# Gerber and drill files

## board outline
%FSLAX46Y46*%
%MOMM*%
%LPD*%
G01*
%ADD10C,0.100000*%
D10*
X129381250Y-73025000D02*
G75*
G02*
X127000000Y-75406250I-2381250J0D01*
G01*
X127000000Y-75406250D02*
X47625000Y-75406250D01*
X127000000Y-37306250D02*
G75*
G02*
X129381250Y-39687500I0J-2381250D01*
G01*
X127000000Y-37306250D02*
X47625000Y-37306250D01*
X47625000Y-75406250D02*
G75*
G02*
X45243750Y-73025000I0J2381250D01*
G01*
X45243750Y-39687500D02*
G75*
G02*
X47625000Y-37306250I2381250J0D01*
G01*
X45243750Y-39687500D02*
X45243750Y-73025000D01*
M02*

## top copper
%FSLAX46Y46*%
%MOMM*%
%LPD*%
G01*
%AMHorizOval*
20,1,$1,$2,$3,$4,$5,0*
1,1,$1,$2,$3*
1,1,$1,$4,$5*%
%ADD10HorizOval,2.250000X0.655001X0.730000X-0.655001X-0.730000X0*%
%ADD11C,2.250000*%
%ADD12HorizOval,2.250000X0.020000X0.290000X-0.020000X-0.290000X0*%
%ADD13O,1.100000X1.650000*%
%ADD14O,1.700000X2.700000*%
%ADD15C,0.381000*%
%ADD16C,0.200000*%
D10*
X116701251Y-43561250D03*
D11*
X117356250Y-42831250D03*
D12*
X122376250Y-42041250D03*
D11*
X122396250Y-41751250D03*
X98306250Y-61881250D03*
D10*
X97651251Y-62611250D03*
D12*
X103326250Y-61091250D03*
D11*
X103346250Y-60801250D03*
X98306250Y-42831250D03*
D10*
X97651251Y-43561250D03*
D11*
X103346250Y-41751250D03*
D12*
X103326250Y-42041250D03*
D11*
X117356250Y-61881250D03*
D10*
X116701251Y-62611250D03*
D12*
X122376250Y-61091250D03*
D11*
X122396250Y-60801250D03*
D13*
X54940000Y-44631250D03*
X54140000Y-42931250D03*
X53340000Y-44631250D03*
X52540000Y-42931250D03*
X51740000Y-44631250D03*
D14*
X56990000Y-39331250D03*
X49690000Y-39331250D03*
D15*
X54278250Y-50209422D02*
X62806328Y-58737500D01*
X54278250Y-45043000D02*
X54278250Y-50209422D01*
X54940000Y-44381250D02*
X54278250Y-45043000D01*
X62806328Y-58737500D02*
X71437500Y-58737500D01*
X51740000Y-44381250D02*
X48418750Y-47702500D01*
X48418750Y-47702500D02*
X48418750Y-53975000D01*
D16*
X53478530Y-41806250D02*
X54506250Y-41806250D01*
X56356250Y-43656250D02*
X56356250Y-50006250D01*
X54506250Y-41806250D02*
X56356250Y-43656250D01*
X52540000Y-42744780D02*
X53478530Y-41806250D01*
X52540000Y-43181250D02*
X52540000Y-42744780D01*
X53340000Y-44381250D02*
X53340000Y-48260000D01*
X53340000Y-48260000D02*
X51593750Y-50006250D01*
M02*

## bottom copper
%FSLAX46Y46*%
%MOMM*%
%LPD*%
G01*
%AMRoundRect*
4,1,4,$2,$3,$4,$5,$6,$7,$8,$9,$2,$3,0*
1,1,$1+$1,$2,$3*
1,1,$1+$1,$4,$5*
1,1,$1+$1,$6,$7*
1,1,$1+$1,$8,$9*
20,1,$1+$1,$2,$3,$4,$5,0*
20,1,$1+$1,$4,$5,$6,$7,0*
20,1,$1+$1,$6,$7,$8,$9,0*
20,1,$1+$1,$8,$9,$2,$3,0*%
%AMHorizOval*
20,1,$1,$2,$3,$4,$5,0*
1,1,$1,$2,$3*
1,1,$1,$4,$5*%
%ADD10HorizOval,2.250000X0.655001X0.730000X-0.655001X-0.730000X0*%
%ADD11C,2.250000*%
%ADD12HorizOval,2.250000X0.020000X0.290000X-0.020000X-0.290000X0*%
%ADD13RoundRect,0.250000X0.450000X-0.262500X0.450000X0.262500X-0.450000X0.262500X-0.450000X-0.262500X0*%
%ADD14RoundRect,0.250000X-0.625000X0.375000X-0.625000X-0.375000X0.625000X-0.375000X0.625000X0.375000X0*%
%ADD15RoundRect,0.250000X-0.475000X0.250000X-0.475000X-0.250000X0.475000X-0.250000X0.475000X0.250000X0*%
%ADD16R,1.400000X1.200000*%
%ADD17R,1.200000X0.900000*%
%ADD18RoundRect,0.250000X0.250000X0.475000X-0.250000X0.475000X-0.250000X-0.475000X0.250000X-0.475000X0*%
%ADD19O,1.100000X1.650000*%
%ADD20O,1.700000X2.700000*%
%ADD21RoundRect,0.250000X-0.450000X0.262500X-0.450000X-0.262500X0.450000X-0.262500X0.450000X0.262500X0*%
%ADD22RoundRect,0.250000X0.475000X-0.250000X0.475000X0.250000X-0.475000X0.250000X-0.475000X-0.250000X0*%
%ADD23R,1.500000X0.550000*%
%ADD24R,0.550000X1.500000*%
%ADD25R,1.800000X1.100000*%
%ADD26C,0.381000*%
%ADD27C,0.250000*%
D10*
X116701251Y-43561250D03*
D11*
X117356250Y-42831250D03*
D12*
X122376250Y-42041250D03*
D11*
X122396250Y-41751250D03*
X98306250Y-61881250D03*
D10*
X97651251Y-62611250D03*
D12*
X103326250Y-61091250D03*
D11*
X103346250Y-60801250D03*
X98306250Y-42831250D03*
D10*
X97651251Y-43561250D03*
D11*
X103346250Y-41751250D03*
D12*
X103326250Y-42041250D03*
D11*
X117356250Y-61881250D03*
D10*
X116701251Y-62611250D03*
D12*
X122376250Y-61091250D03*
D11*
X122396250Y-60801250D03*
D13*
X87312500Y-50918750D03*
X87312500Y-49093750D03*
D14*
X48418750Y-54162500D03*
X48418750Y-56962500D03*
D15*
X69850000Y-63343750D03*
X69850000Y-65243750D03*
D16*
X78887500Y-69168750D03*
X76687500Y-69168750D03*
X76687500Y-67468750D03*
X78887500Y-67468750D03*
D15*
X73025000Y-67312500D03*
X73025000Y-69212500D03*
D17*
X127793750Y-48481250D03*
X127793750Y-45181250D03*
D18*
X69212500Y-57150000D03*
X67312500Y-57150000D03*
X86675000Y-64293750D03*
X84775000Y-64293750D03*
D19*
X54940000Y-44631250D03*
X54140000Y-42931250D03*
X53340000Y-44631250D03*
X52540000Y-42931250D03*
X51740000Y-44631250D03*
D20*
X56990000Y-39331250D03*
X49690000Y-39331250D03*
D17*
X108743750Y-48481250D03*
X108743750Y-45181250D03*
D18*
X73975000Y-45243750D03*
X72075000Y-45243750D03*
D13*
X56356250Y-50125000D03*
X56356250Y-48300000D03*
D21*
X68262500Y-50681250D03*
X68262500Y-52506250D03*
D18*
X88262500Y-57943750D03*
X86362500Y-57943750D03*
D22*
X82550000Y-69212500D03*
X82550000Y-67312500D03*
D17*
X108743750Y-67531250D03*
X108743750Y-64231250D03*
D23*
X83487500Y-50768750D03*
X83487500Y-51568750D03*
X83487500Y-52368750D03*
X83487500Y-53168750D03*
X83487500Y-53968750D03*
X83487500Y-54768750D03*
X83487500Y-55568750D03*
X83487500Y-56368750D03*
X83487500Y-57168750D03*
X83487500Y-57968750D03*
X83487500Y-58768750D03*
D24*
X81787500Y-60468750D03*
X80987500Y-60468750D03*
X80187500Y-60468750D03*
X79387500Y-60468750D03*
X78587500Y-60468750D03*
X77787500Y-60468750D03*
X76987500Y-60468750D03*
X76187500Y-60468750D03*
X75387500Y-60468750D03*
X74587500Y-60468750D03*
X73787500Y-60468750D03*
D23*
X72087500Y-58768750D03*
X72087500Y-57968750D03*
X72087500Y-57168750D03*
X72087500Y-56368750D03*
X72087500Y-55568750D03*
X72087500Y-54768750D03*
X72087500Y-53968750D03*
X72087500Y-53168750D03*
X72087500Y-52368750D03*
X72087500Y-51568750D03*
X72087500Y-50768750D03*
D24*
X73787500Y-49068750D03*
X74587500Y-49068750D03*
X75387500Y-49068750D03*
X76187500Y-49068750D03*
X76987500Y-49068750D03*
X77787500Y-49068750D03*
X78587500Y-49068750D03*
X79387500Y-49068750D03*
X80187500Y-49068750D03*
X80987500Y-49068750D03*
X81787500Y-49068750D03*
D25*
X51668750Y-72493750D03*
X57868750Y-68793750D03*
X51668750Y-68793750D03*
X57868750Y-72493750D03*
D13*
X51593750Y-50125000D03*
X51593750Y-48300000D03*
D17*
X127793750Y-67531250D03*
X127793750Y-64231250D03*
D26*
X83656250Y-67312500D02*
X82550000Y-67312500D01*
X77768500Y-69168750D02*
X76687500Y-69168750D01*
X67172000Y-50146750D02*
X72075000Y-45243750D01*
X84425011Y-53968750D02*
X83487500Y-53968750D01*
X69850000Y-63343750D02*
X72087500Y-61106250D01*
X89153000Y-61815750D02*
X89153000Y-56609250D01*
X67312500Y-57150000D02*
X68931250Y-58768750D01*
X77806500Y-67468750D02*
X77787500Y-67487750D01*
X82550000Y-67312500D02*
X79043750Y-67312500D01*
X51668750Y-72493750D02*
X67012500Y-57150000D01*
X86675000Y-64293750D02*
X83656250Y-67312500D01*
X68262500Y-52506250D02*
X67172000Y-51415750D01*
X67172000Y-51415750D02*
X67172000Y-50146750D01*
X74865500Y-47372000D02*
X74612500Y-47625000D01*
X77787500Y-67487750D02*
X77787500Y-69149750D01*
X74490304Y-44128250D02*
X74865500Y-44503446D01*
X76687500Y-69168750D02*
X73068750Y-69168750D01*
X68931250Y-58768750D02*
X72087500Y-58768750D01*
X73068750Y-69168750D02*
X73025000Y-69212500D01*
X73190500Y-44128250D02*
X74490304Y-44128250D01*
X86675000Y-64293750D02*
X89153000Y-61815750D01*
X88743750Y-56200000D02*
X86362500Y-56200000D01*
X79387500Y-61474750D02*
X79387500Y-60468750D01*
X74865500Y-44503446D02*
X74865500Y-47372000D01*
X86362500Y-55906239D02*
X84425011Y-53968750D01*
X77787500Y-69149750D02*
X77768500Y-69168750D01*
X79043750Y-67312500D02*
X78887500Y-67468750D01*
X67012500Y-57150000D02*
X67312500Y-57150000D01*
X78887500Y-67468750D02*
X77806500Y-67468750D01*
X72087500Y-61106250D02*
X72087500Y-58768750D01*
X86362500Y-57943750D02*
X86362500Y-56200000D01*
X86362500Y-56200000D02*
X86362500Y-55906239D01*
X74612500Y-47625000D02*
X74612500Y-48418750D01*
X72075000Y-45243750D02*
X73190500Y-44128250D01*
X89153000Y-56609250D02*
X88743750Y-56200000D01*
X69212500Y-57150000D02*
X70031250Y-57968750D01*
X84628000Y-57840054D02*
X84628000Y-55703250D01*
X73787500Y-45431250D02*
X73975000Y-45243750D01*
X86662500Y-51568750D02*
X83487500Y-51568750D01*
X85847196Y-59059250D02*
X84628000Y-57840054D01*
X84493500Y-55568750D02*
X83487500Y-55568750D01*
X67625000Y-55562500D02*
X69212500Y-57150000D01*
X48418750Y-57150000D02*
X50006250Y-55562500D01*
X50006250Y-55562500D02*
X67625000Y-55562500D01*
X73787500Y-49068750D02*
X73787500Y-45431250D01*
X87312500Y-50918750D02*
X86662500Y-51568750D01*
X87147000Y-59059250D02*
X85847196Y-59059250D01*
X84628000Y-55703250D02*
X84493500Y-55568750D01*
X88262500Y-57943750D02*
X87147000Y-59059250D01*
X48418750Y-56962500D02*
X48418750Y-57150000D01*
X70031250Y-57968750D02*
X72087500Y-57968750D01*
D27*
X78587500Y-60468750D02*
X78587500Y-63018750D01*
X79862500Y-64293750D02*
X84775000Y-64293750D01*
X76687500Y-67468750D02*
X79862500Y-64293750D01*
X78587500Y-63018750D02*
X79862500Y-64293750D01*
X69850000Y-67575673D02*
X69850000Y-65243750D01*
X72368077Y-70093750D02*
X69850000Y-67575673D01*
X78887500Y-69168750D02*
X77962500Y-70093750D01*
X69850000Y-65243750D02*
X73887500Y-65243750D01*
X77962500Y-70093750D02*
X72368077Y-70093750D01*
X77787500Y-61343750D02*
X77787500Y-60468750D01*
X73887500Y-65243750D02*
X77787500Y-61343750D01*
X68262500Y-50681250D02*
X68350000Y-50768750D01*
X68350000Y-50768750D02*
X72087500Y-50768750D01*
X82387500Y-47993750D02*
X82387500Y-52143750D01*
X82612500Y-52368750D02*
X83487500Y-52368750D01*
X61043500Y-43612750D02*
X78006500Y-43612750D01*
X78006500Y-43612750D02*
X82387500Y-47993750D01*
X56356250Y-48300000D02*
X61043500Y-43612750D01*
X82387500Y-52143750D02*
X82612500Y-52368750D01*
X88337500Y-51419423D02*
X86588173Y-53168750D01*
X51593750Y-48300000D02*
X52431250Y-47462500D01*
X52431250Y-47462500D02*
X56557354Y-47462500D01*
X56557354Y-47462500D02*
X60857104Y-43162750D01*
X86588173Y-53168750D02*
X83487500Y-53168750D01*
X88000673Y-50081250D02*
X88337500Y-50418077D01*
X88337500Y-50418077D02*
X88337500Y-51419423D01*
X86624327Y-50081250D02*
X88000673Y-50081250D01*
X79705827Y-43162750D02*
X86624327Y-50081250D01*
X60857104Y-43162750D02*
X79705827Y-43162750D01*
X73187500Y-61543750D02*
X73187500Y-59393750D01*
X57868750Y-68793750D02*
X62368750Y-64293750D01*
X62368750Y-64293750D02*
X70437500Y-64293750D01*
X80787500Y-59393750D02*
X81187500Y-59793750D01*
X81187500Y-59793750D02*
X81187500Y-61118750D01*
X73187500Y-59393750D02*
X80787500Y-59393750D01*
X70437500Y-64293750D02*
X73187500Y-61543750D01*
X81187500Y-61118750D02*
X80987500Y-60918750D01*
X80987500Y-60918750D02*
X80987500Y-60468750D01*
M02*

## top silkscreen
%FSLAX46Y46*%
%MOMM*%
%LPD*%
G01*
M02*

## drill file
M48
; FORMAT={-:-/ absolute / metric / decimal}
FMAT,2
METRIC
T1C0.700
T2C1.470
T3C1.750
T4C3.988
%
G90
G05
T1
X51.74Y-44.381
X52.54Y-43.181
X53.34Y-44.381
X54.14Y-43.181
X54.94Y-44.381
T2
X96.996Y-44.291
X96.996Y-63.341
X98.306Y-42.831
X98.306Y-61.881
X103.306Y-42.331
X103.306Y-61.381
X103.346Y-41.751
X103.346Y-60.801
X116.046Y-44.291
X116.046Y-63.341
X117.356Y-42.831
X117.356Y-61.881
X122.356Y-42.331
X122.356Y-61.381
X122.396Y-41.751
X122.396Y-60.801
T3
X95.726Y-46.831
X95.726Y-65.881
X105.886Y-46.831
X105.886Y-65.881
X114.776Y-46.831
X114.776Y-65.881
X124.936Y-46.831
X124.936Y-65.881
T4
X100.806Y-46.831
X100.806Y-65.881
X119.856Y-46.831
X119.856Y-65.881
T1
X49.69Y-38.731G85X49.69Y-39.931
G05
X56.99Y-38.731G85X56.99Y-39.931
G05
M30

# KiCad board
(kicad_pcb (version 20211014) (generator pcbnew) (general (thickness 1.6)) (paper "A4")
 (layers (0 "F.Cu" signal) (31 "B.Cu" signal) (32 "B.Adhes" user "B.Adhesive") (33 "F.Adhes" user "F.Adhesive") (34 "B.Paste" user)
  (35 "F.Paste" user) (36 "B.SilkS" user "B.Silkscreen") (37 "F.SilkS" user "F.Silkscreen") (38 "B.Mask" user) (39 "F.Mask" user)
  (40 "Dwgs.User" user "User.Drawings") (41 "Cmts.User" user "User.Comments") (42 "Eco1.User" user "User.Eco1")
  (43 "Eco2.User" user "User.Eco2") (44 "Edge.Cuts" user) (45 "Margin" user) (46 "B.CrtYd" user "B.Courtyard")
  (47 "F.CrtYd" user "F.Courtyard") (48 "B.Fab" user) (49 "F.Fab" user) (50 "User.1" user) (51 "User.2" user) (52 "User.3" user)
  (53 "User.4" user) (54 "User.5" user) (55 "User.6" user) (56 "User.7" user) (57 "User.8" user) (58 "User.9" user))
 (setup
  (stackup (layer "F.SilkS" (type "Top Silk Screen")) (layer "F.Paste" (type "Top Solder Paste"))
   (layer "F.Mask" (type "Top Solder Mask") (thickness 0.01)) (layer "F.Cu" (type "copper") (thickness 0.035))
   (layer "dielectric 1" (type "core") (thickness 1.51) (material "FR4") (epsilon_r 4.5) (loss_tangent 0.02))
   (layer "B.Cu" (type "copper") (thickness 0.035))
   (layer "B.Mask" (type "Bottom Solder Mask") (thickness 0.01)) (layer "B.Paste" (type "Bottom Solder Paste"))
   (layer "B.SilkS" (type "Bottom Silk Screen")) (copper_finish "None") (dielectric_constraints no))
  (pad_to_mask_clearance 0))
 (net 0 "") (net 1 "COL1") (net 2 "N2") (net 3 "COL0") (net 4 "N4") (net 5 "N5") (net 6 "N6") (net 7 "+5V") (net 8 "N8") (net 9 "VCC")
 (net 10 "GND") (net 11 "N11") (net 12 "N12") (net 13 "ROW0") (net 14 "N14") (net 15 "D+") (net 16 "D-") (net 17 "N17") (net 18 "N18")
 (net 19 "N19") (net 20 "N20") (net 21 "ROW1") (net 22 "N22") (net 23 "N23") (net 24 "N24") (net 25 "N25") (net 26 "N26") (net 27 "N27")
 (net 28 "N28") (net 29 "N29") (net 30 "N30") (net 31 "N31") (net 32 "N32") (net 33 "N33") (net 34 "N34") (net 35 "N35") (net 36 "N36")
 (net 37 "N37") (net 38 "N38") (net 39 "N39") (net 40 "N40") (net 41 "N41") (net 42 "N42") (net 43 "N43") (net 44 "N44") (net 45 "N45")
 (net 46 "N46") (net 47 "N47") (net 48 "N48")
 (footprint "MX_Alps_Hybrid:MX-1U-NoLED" (layer "F.Cu") (at 119.85625 46.83125)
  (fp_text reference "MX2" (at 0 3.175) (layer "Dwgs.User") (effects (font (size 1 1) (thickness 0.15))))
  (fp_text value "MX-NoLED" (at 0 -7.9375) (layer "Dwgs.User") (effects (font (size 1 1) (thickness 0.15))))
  (pad "" np_thru_hole circle locked (at 5.08 0 48.0996) (size 1.75 1.75) (drill 1.75) (layers *.Cu *.Mask))
  (pad "" np_thru_hole circle locked (at 0 0) (size 3.9878 3.9878) (drill 3.9878) (layers *.Cu *.Mask))
  (pad "" np_thru_hole circle locked (at -5.08 0 48.0996) (size 1.75 1.75) (drill 1.75) (layers *.Cu *.Mask))
  (pad "1" thru_hole oval locked (at -3.81 -2.54 48.0996) (size 4.211556 2.25) (drill 1.47 (offset 0.980778 0)) (layers *.Cu "B.Mask")
   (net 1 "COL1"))
  (pad "1" thru_hole circle locked (at -2.5 -4) (size 2.25 2.25) (drill 1.47) (layers *.Cu "B.Mask") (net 1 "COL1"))
  (pad "2" thru_hole oval locked (at 2.5 -4.5 86.0548) (size 2.831378 2.25) (drill 1.47 (offset 0.290689 0)) (layers *.Cu "B.Mask")
   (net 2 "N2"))
  (pad "2" thru_hole circle locked (at 2.54 -5.08) (size 2.25 2.25) (drill 1.47) (layers *.Cu "B.Mask") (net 2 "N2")))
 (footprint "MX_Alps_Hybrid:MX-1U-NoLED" (layer "F.Cu") (at 100.80625 65.88125)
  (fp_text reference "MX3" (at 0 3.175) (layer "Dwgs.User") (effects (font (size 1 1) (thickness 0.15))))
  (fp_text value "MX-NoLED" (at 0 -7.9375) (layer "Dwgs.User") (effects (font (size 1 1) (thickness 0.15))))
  (pad "" np_thru_hole circle locked (at 5.08 0 48.0996) (size 1.75 1.75) (drill 1.75) (layers *.Cu *.Mask))
  (pad "" np_thru_hole circle locked (at 0 0) (size 3.9878 3.9878) (drill 3.9878) (layers *.Cu *.Mask))
  (pad "" np_thru_hole circle locked (at -5.08 0 48.0996) (size 1.75 1.75) (drill 1.75) (layers *.Cu *.Mask))
  (pad "1" thru_hole circle locked (at -2.5 -4) (size 2.25 2.25) (drill 1.47) (layers *.Cu "B.Mask") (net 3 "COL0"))
  (pad "1" thru_hole oval locked (at -3.81 -2.54 48.0996) (size 4.211556 2.25) (drill 1.47 (offset 0.980778 0)) (layers *.Cu "B.Mask")
   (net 3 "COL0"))
  (pad "2" thru_hole oval locked (at 2.5 -4.5 86.0548) (size 2.831378 2.25) (drill 1.47 (offset 0.290689 0)) (layers *.Cu "B.Mask")
   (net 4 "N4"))
  (pad "2" thru_hole circle locked (at 2.54 -5.08) (size 2.25 2.25) (drill 1.47) (layers *.Cu "B.Mask") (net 4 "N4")))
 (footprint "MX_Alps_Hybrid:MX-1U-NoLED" (layer "F.Cu") (at 100.80625 46.83125)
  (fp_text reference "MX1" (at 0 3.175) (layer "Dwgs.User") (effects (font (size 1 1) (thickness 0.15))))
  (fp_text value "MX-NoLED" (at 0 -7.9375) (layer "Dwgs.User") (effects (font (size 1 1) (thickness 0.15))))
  (pad "" np_thru_hole circle locked (at 0 0) (size 3.9878 3.9878) (drill 3.9878) (layers *.Cu *.Mask))
  (pad "" np_thru_hole circle locked (at -5.08 0 48.0996) (size 1.75 1.75) (drill 1.75) (layers *.Cu *.Mask))
  (pad "" np_thru_hole circle locked (at 5.08 0 48.0996) (size 1.75 1.75) (drill 1.75) (layers *.Cu *.Mask))
  (pad "1" thru_hole circle locked (at -2.5 -4) (size 2.25 2.25) (drill 1.47) (layers *.Cu "B.Mask") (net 3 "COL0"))
  (pad "1" thru_hole oval locked (at -3.81 -2.54 48.0996) (size 4.211556 2.25) (drill 1.47 (offset 0.980778 0)) (layers *.Cu "B.Mask")
   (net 3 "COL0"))
  (pad "2" thru_hole circle locked (at 2.54 -5.08) (size 2.25 2.25) (drill 1.47) (layers *.Cu "B.Mask") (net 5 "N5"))
  (pad "2" thru_hole oval locked (at 2.5 -4.5 86.0548) (size 2.831378 2.25) (drill 1.47 (offset 0.290689 0)) (layers *.Cu "B.Mask")
   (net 5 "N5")))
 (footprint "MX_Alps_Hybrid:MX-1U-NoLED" (layer "F.Cu") (at 119.85625 65.88125)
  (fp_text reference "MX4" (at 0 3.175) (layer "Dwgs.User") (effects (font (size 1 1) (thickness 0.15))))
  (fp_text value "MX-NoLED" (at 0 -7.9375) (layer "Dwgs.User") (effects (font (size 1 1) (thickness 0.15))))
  (pad "" np_thru_hole circle locked (at 5.08 0 48.0996) (size 1.75 1.75) (drill 1.75) (layers *.Cu *.Mask))
  (pad "" np_thru_hole circle locked (at -5.08 0 48.0996) (size 1.75 1.75) (drill 1.75) (layers *.Cu *.Mask))
  (pad "" np_thru_hole circle locked (at 0 0) (size 3.9878 3.9878) (drill 3.9878) (layers *.Cu *.Mask))
  (pad "1" thru_hole circle locked (at -2.5 -4) (size 2.25 2.25) (drill 1.47) (layers *.Cu "B.Mask") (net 1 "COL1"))
  (pad "1" thru_hole oval locked (at -3.81 -2.54 48.0996) (size 4.211556 2.25) (drill 1.47 (offset 0.980778 0)) (layers *.Cu "B.Mask")
   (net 1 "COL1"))
  (pad "2" thru_hole oval locked (at 2.5 -4.5 86.0548) (size 2.831378 2.25) (drill 1.47 (offset 0.290689 0)) (layers *.Cu "B.Mask")
   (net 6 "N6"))
  (pad "2" thru_hole circle locked (at 2.54 -5.08) (size 2.25 2.25) (drill 1.47) (layers *.Cu "B.Mask") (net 6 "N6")))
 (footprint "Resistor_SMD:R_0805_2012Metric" (layer "B.Cu") (at 87.3125 50.00625 90)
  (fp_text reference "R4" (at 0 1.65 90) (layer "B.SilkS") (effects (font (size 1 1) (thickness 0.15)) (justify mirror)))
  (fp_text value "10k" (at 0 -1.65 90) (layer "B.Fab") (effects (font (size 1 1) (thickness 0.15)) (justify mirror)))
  (pad "1" smd roundrect (at -0.9125 0 90) (size 1.025 1.4) (layers "B.Cu" "B.Paste" "B.Mask") (roundrect_rratio 0.243902) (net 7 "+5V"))
  (pad "2" smd roundrect (at 0.9125 0 90) (size 1.025 1.4) (layers "B.Cu" "B.Paste" "B.Mask") (roundrect_rratio 0.243902) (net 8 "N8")))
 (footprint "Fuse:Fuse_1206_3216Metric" (layer "B.Cu") (at 48.41875 55.5625 -90)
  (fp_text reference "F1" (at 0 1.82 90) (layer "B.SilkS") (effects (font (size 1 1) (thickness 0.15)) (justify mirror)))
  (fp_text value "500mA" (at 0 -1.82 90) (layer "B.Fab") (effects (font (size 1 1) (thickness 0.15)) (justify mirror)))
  (pad "1" smd roundrect (at -1.4 0 270) (size 1.25 1.75) (layers "B.Cu" "B.Paste" "B.Mask") (roundrect_rratio 0.2) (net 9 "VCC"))
  (pad "2" smd roundrect (at 1.4 0 270) (size 1.25 1.75) (layers "B.Cu" "B.Paste" "B.Mask") (roundrect_rratio 0.2) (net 7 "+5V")))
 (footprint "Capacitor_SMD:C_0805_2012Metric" (layer "B.Cu") (at 69.85 64.29375 -90)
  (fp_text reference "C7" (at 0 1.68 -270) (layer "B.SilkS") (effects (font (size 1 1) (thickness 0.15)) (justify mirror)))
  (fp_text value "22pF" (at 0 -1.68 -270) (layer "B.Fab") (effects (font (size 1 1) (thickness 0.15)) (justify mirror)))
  (pad "1" smd roundrect (at -0.95 0 270) (size 1 1.45) (layers "B.Cu" "B.Paste" "B.Mask") (roundrect_rratio 0.25) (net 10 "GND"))
  (pad "2" smd roundrect (at 0.95 0 270) (size 1 1.45) (layers "B.Cu" "B.Paste" "B.Mask") (roundrect_rratio 0.25) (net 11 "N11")))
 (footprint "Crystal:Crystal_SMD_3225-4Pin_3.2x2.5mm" (layer "B.Cu") (at 77.7875 68.31875 180)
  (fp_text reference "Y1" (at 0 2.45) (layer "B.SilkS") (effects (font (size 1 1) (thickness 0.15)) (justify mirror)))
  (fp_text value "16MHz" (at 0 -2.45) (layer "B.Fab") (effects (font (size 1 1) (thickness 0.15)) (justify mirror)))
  (pad "1" smd rect (at -1.1 -0.85 180) (size 1.4 1.2) (layers "B.Cu" "B.Paste" "B.Mask") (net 11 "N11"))
  (pad "2" smd rect (at 1.1 -0.85 180) (size 1.4 1.2) (layers "B.Cu" "B.Paste" "B.Mask") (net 10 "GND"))
  (pad "3" smd rect (at 1.1 0.85 180) (size 1.4 1.2) (layers "B.Cu" "B.Paste" "B.Mask") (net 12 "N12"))
  (pad "4" smd rect (at -1.1 0.85 180) (size 1.4 1.2) (layers "B.Cu" "B.Paste" "B.Mask") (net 10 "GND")))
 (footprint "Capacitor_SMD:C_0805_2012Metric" (layer "B.Cu") (at 73.025 68.2625 -90)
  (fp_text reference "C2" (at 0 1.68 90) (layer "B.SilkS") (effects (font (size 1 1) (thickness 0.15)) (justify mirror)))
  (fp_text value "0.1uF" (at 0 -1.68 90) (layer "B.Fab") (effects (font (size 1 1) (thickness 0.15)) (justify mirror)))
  (pad "1" smd roundrect (at -0.95 0 270) (size 1 1.45) (layers "B.Cu" "B.Paste" "B.Mask") (roundrect_rratio 0.25) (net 7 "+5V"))
  (pad "2" smd roundrect (at 0.95 0 270) (size 1 1.45) (layers "B.Cu" "B.Paste" "B.Mask") (roundrect_rratio 0.25) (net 10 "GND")))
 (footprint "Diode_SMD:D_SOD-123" (layer "B.Cu") (at 127.79375 46.83125 90)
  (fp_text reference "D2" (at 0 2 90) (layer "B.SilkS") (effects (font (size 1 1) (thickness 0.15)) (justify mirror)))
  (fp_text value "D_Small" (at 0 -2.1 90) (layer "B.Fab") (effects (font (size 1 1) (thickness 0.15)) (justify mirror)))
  (pad "1" smd rect (at -1.65 0 90) (size 0.9 1.2) (layers "B.Cu" "B.Paste" "B.Mask") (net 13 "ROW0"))
  (pad "2" smd rect (at 1.65 0 90) (size 0.9 1.2) (layers "B.Cu" "B.Paste" "B.Mask") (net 2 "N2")))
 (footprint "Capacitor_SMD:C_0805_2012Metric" (layer "B.Cu") (at 68.2625 57.15 180)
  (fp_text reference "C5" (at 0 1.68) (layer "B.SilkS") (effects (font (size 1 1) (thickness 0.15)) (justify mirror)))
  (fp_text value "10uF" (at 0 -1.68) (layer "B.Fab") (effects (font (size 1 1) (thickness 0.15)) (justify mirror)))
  (pad "1" smd roundrect (at -0.95 0 180) (size 1 1.45) (layers "B.Cu" "B.Paste" "B.Mask") (roundrect_rratio 0.25) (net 7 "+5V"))
  (pad "2" smd roundrect (at 0.95 0 180) (size 1 1.45) (layers "B.Cu" "B.Paste" "B.Mask") (roundrect_rratio 0.25) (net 10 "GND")))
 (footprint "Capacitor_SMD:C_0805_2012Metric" (layer "B.Cu") (at 85.725 64.29375 180)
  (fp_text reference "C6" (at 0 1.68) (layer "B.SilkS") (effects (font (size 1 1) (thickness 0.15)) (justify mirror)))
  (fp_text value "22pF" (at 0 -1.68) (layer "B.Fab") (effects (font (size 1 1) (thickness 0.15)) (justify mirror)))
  (pad "1" smd roundrect (at -0.95 0 180) (size 1 1.45) (layers "B.Cu" "B.Paste" "B.Mask") (roundrect_rratio 0.25) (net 10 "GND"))
  (pad "2" smd roundrect (at 0.95 0 180) (size 1 1.45) (layers "B.Cu" "B.Paste" "B.Mask") (roundrect_rratio 0.25) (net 12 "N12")))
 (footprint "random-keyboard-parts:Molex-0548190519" (layer "B.Cu") (at 53.34 37.58125 -90)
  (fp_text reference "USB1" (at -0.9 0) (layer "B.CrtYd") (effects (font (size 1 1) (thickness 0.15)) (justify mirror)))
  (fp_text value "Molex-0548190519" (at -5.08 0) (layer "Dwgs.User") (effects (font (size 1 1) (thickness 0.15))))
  (pad "1" thru_hole oval locked (at 6.8 -1.6 270) (size 1.65 1.1) (drill oval 0.7 (offset 0.25 0)) (layers *.Cu "F.Mask") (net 10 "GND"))
  (pad "2" thru_hole oval locked (at 5.6 -0.8 90) (size 1.65 1.1) (drill oval 0.7 (offset 0.25 0)) (layers *.Cu "F.Mask") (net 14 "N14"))
  (pad "3" thru_hole oval locked (at 6.8 0 270) (size 1.65 1.1) (drill oval 0.7 (offset 0.25 0)) (layers *.Cu "F.Mask") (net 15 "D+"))
  (pad "4" thru_hole oval locked (at 5.6 0.8 90) (size 1.65 1.1) (drill oval 0.7 (offset 0.25 0)) (layers *.Cu "F.Mask") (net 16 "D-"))
  (pad "5" thru_hole oval locked (at 6.8 1.6 270) (size 1.65 1.1) (drill oval 0.7 (offset 0.25 0)) (layers *.Cu "F.Mask") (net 9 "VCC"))
  (pad "6" thru_hole oval locked (at 1.75 -3.65 270) (size 2.7 1.7) (drill oval 1.9 0.7) (layers *.Cu *.Mask) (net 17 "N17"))
  (pad "6" thru_hole oval locked (at 1.75 3.65 270) (size 2.7 1.7) (drill oval 1.9 0.7) (layers *.Cu *.Mask) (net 17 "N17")))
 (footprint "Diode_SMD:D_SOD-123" (layer "B.Cu") (at 108.74375 46.83125 90)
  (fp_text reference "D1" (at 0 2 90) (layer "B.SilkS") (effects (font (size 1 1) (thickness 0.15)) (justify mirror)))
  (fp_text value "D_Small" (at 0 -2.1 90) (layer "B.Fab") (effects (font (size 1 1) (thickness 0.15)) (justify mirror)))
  (pad "1" smd rect (at -1.65 0 90) (size 0.9 1.2) (layers "B.Cu" "B.Paste" "B.Mask") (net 13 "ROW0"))
  (pad "2" smd rect (at 1.65 0 90) (size 0.9 1.2) (layers "B.Cu" "B.Paste" "B.Mask") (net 5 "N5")))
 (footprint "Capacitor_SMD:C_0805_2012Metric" (layer "B.Cu") (at 73.025 45.24375 180)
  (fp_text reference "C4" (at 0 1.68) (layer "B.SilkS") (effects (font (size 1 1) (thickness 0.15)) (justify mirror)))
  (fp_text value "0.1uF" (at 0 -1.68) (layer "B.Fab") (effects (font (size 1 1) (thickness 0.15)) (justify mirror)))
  (pad "1" smd roundrect (at -0.95 0 180) (size 1 1.45) (layers "B.Cu" "B.Paste" "B.Mask") (roundrect_rratio 0.25) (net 7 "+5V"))
  (pad "2" smd roundrect (at 0.95 0 180) (size 1 1.45) (layers "B.Cu" "B.Paste" "B.Mask") (roundrect_rratio 0.25) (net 10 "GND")))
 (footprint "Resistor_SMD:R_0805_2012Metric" (layer "B.Cu") (at 56.35625 49.2125 90)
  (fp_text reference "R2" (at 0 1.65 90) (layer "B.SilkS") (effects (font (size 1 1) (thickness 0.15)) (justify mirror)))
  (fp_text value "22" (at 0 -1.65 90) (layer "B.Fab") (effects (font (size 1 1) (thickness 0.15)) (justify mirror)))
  (pad "1" smd roundrect (at -0.9125 0 90) (size 1.025 1.4) (layers "B.Cu" "B.Paste" "B.Mask") (roundrect_rratio 0.243902) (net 16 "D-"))
  (pad "2" smd roundrect (at 0.9125 0 90) (size 1.025 1.4) (layers "B.Cu" "B.Paste" "B.Mask") (roundrect_rratio 0.243902) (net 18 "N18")))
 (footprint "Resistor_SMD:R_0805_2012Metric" (layer "B.Cu") (at 68.2625 51.59375 -90)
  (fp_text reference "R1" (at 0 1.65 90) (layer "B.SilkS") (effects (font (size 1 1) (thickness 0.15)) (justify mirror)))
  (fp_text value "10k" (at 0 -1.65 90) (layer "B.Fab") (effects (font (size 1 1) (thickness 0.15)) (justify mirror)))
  (pad "1" smd roundrect (at -0.9125 0 270) (size 1.025 1.4) (layers "B.Cu" "B.Paste" "B.Mask") (roundrect_rratio 0.243902) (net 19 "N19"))
  (pad "2" smd roundrect (at 0.9125 0 270) (size 1.025 1.4) (layers "B.Cu" "B.Paste" "B.Mask") (roundrect_rratio 0.243902) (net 10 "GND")))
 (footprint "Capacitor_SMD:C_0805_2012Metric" (layer "B.Cu") (at 87.3125 57.94375 180)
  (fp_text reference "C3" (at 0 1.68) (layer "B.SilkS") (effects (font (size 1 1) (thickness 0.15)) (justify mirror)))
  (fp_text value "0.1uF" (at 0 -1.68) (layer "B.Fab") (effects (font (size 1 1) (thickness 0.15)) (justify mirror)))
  (pad "1" smd roundrect (at -0.95 0 180) (size 1 1.45) (layers "B.Cu" "B.Paste" "B.Mask") (roundrect_rratio 0.25) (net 7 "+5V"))
  (pad "2" smd roundrect (at 0.95 0 180) (size 1 1.45) (layers "B.Cu" "B.Paste" "B.Mask") (roundrect_rratio 0.25) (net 10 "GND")))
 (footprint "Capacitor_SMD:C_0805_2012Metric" (layer "B.Cu") (at 82.55 68.2625 90)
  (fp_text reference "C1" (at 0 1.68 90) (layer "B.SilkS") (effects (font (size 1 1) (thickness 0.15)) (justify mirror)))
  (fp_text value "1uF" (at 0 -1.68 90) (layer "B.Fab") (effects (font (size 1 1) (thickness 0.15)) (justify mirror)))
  (pad "1" smd roundrect (at -0.95 0 90) (size 1 1.45) (layers "B.Cu" "B.Paste" "B.Mask") (roundrect_rratio 0.25) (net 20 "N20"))
  (pad "2" smd roundrect (at 0.95 0 90) (size 1 1.45) (layers "B.Cu" "B.Paste" "B.Mask") (roundrect_rratio 0.25) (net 10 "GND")))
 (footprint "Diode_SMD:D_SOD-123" (layer "B.Cu") (at 108.74375 65.88125 90)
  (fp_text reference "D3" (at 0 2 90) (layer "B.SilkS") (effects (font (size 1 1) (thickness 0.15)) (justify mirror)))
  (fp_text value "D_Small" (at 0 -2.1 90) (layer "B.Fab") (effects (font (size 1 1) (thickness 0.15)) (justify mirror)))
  (pad "1" smd rect (at -1.65 0 90) (size 0.9 1.2) (layers "B.Cu" "B.Paste" "B.Mask") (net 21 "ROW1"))
  (pad "2" smd rect (at 1.65 0 90) (size 0.9 1.2) (layers "B.Cu" "B.Paste" "B.Mask") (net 4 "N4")))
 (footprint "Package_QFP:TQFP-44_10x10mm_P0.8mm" (layer "B.Cu") (at 77.7875 54.76875 180)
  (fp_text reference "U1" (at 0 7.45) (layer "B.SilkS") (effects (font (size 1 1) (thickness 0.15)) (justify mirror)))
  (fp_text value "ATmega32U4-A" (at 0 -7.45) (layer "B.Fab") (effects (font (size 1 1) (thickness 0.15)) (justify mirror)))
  (pad "1" smd rect (at -5.7 4 180) (size 1.5 0.55) (layers "B.Cu" "B.Paste" "B.Mask") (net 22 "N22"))
  (pad "2" smd rect (at -5.7 3.2 180) (size 1.5 0.55) (layers "B.Cu" "B.Paste" "B.Mask") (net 7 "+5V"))
  (pad "3" smd rect (at -5.7 2.4 180) (size 1.5 0.55) (layers "B.Cu" "B.Paste" "B.Mask") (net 18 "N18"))
  (pad "4" smd rect (at -5.7 1.6 180) (size 1.5 0.55) (layers "B.Cu" "B.Paste" "B.Mask") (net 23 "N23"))
  (pad "5" smd rect (at -5.7 0.8 180) (size 1.5 0.55) (layers "B.Cu" "B.Paste" "B.Mask") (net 10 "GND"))
  (pad "6" smd rect (at -5.7 0 180) (size 1.5 0.55) (layers "B.Cu" "B.Paste" "B.Mask") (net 20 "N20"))
  (pad "7" smd rect (at -5.7 -0.8 180) (size 1.5 0.55) (layers "B.Cu" "B.Paste" "B.Mask") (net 7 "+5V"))
  (pad "8" smd rect (at -5.7 -1.6 180) (size 1.5 0.55) (layers "B.Cu" "B.Paste" "B.Mask") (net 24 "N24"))
  (pad "9" smd rect (at -5.7 -2.4 180) (size 1.5 0.55) (layers "B.Cu" "B.Paste" "B.Mask") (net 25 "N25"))
  (pad "10" smd rect (at -5.7 -3.2 180) (size 1.5 0.55) (layers "B.Cu" "B.Paste" "B.Mask") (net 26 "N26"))
  (pad "11" smd rect (at -5.7 -4 180) (size 1.5 0.55) (layers "B.Cu" "B.Paste" "B.Mask") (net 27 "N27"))
  (pad "12" smd rect (at -4 -5.7 90) (size 1.5 0.55) (layers "B.Cu" "B.Paste" "B.Mask") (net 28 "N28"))
  (pad "13" smd rect (at -3.2 -5.7 90) (size 1.5 0.55) (layers "B.Cu" "B.Paste" "B.Mask") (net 8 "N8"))
  (pad "14" smd rect (at -2.4 -5.7 90) (size 1.5 0.55) (layers "B.Cu" "B.Paste" "B.Mask") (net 7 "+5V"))
  (pad "15" smd rect (at -1.6 -5.7 90) (size 1.5 0.55) (layers "B.Cu" "B.Paste" "B.Mask") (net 10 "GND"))
  (pad "16" smd rect (at -0.8 -5.7 90) (size 1.5 0.55) (layers "B.Cu" "B.Paste" "B.Mask") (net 12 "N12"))
  (pad "17" smd rect (at 0 -5.7 90) (size 1.5 0.55) (layers "B.Cu" "B.Paste" "B.Mask") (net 11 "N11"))
  (pad "18" smd rect (at 0.8 -5.7 90) (size 1.5 0.55) (layers "B.Cu" "B.Paste" "B.Mask") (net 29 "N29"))
  (pad "19" smd rect (at 1.6 -5.7 90) (size 1.5 0.55) (layers "B.Cu" "B.Paste" "B.Mask") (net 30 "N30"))
  (pad "20" smd rect (at 2.4 -5.7 90) (size 1.5 0.55) (layers "B.Cu" "B.Paste" "B.Mask") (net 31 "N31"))
  (pad "21" smd rect (at 3.2 -5.7 90) (size 1.5 0.55) (layers "B.Cu" "B.Paste" "B.Mask") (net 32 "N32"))
  (pad "22" smd rect (at 4 -5.7 90) (size 1.5 0.55) (layers "B.Cu" "B.Paste" "B.Mask") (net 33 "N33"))
  (pad "23" smd rect (at 5.7 -4 180) (size 1.5 0.55) (layers "B.Cu" "B.Paste" "B.Mask") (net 10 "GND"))
  (pad "24" smd rect (at 5.7 -3.2 180) (size 1.5 0.55) (layers "B.Cu" "B.Paste" "B.Mask") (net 7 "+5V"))
  (pad "25" smd rect (at 5.7 -2.4 180) (size 1.5 0.55) (layers "B.Cu" "B.Paste" "B.Mask") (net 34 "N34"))
  (pad "26" smd rect (at 5.7 -1.6 180) (size 1.5 0.55) (layers "B.Cu" "B.Paste" "B.Mask") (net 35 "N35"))
  (pad "27" smd rect (at 5.7 -0.8 180) (size 1.5 0.55) (layers "B.Cu" "B.Paste" "B.Mask") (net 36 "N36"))
  (pad "28" smd rect (at 5.7 0 180) (size 1.5 0.55) (layers "B.Cu" "B.Paste" "B.Mask") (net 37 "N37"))
  (pad "29" smd rect (at 5.7 0.8 180) (size 1.5 0.55) (layers "B.Cu" "B.Paste" "B.Mask") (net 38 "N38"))
  (pad "30" smd rect (at 5.7 1.6 180) (size 1.5 0.55) (layers "B.Cu" "B.Paste" "B.Mask") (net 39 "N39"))
  (pad "31" smd rect (at 5.7 2.4 180) (size 1.5 0.55) (layers "B.Cu" "B.Paste" "B.Mask") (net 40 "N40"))
  (pad "32" smd rect (at 5.7 3.2 180) (size 1.5 0.55) (layers "B.Cu" "B.Paste" "B.Mask") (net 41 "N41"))
  (pad "33" smd rect (at 5.7 4 180) (size 1.5 0.55) (layers "B.Cu" "B.Paste" "B.Mask") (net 19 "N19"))
  (pad "34" smd rect (at 4 5.7 90) (size 1.5 0.55) (layers "B.Cu" "B.Paste" "B.Mask") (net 7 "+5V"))
  (pad "35" smd rect (at 3.2 5.7 90) (size 1.5 0.55) (layers "B.Cu" "B.Paste" "B.Mask") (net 10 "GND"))
  (pad "36" smd rect (at 2.4 5.7 90) (size 1.5 0.55) (layers "B.Cu" "B.Paste" "B.Mask") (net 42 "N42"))
  (pad "37" smd rect (at 1.6 5.7 90) (size 1.5 0.55) (layers "B.Cu" "B.Paste" "B.Mask") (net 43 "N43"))
  (pad "38" smd rect (at 0.8 5.7 90) (size 1.5 0.55) (layers "B.Cu" "B.Paste" "B.Mask") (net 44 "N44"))
  (pad "39" smd rect (at 0 5.7 90) (size 1.5 0.55) (layers "B.Cu" "B.Paste" "B.Mask") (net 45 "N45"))
  (pad "40" smd rect (at -0.8 5.7 90) (size 1.5 0.55) (layers "B.Cu" "B.Paste" "B.Mask") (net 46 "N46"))
  (pad "41" smd rect (at -1.6 5.7 90) (size 1.5 0.55) (layers "B.Cu" "B.Paste" "B.Mask") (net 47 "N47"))
  (pad "42" smd rect (at -2.4 5.7 90) (size 1.5 0.55) (layers "B.Cu" "B.Paste" "B.Mask") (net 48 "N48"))
  (pad "43" smd rect (at -3.2 5.7 90) (size 1.5 0.55) (layers "B.Cu" "B.Paste" "B.Mask") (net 10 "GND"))
  (pad "44" smd rect (at -4 5.7 90) (size 1.5 0.55) (layers "B.Cu" "B.Paste" "B.Mask") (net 7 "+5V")))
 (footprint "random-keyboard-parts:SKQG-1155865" (layer "B.Cu") (at 54.76875 70.64375 180)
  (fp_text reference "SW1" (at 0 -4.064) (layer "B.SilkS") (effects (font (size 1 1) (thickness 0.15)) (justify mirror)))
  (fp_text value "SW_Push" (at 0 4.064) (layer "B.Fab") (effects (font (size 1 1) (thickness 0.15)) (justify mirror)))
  (pad "1" smd rect locked (at 3.1 -1.85 180) (size 1.8 1.1) (layers "B.Cu" "B.Paste" "B.Mask") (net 10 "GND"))
  (pad "2" smd rect locked (at -3.1 1.85 180) (size 1.8 1.1) (layers "B.Cu" "B.Paste" "B.Mask") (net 8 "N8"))
  (pad "3" smd rect locked (at 3.1 1.85 180) (size 1.8 1.1) (layers "B.Cu" "B.Paste" "B.Mask"))
  (pad "4" smd rect locked (at -3.1 -1.85 180) (size 1.8 1.1) (layers "B.Cu" "B.Paste" "B.Mask")))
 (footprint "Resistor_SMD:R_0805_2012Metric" (layer "B.Cu") (at 51.59375 49.2125 90)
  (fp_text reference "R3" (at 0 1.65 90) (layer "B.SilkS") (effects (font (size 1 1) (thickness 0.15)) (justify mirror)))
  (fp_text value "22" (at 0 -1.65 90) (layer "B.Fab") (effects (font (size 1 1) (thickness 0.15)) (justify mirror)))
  (pad "1" smd roundrect (at -0.9125 0 90) (size 1.025 1.4) (layers "B.Cu" "B.Paste" "B.Mask") (roundrect_rratio 0.243902) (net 15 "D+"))
  (pad "2" smd roundrect (at 0.9125 0 90) (size 1.025 1.4) (layers "B.Cu" "B.Paste" "B.Mask") (roundrect_rratio 0.243902) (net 23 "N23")))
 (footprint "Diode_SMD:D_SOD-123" (layer "B.Cu") (at 127.79375 65.88125 90)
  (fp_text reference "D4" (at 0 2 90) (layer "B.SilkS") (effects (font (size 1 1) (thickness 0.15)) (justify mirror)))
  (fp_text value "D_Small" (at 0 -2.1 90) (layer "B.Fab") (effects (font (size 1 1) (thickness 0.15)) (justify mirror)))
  (pad "1" smd rect (at -1.65 0 90) (size 0.9 1.2) (layers "B.Cu" "B.Paste" "B.Mask") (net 21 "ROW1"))
  (pad "2" smd rect (at 1.65 0 90) (size 0.9 1.2) (layers "B.Cu" "B.Paste" "B.Mask") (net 6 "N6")))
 (gr_arc (start 129.38125 73.025) (mid 128.683798 74.708798) (end 127 75.40625) (layer "Edge.Cuts") (width 0.1))
 (gr_line (start 127 75.40625) (end 47.625 75.40625) (layer "Edge.Cuts") (width 0.1))
 (gr_arc (start 127 37.30625) (mid 128.683798 38.003702) (end 129.38125 39.6875) (layer "Edge.Cuts") (width 0.1))
 (gr_line (start 127 37.30625) (end 47.625 37.30625) (layer "Edge.Cuts") (width 0.1))
 (gr_arc (start 47.625 75.40625) (mid 45.941202 74.708798) (end 45.24375 73.025) (layer "Edge.Cuts") (width 0.1))
 (gr_arc (start 45.24375 39.6875) (mid 45.941202 38.003702) (end 47.625 37.30625) (layer "Edge.Cuts") (width 0.1))
 (gr_line (start 45.24375 39.6875) (end 45.24375 73.025) (layer "Edge.Cuts") (width 0.1))
 (segment (start 54.27825 50.209422) (end 62.806328 58.7375) (width 0.381) (layer "F.Cu") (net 10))
 (segment (start 54.27825 45.043) (end 54.27825 50.209422) (width 0.381) (layer "F.Cu") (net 10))
 (segment (start 54.94 44.38125) (end 54.27825 45.043) (width 0.381) (layer "F.Cu") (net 10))
 (segment (start 62.806328 58.7375) (end 71.4375 58.7375) (width 0.381) (layer "F.Cu") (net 10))
 (segment (start 83.65625 67.3125) (end 82.55 67.3125) (width 0.381) (layer "B.Cu") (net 10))
 (segment (start 77.7685 69.16875) (end 76.6875 69.16875) (width 0.381) (layer "B.Cu") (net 10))
 (segment (start 67.172 50.14675) (end 72.075 45.24375) (width 0.381) (layer "B.Cu") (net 10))
 (segment (start 84.425011 53.96875) (end 83.4875 53.96875) (width 0.381) (layer "B.Cu") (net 10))
 (segment (start 69.85 63.34375) (end 72.0875 61.10625) (width 0.381) (layer "B.Cu") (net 10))
 (segment (start 89.153 61.81575) (end 89.153 56.60925) (width 0.381) (layer "B.Cu") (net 10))
 (segment (start 67.3125 57.15) (end 68.93125 58.76875) (width 0.381) (layer "B.Cu") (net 10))
 (segment (start 77.8065 67.46875) (end 77.7875 67.48775) (width 0.381) (layer "B.Cu") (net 10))
 (segment (start 82.55 67.3125) (end 79.04375 67.3125) (width 0.381) (layer "B.Cu") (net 10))
 (segment (start 51.66875 72.49375) (end 67.0125 57.15) (width 0.381) (layer "B.Cu") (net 10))
 (segment (start 86.675 64.29375) (end 83.65625 67.3125) (width 0.381) (layer "B.Cu") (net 10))
 (segment (start 68.2625 52.50625) (end 67.172 51.41575) (width 0.381) (layer "B.Cu") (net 10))
 (segment (start 67.172 51.41575) (end 67.172 50.14675) (width 0.381) (layer "B.Cu") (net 10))
 (segment (start 74.8655 47.372) (end 74.6125 47.625) (width 0.381) (layer "B.Cu") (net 10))
 (segment (start 77.7875 67.48775) (end 77.7875 69.14975) (width 0.381) (layer "B.Cu") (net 10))
 (segment (start 74.490304 44.12825) (end 74.8655 44.503446) (width 0.381) (layer "B.Cu") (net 10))
 (segment (start 76.6875 69.16875) (end 73.06875 69.16875) (width 0.381) (layer "B.Cu") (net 10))
 (segment (start 68.93125 58.76875) (end 72.0875 58.76875) (width 0.381) (layer "B.Cu") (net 10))
 (segment (start 73.06875 69.16875) (end 73.025 69.2125) (width 0.381) (layer "B.Cu") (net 10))
 (segment (start 73.1905 44.12825) (end 74.490304 44.12825) (width 0.381) (layer "B.Cu") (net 10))
 (segment (start 86.675 64.29375) (end 89.153 61.81575) (width 0.381) (layer "B.Cu") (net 10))
 (segment (start 88.74375 56.2) (end 86.3625 56.2) (width 0.381) (layer "B.Cu") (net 10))
 (segment (start 79.3875 61.47475) (end 79.3875 60.46875) (width 0.381) (layer "B.Cu") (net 10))
 (segment (start 74.8655 44.503446) (end 74.8655 47.372) (width 0.381) (layer "B.Cu") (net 10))
 (segment (start 86.3625 55.906239) (end 84.425011 53.96875) (width 0.381) (layer "B.Cu") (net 10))
 (segment (start 77.7875 69.14975) (end 77.7685 69.16875) (width 0.381) (layer "B.Cu") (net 10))
 (segment (start 79.04375 67.3125) (end 78.8875 67.46875) (width 0.381) (layer "B.Cu") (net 10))
 (segment (start 67.0125 57.15) (end 67.3125 57.15) (width 0.381) (layer "B.Cu") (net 10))
 (segment (start 78.8875 67.46875) (end 77.8065 67.46875) (width 0.381) (layer "B.Cu") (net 10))
 (segment (start 72.0875 61.10625) (end 72.0875 58.76875) (width 0.381) (layer "B.Cu") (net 10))
 (segment (start 86.3625 57.94375) (end 86.3625 56.2) (width 0.381) (layer "B.Cu") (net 10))
 (segment (start 86.3625 56.2) (end 86.3625 55.906239) (width 0.381) (layer "B.Cu") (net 10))
 (segment (start 74.6125 47.625) (end 74.6125 48.41875) (width 0.381) (layer "B.Cu") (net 10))
 (segment (start 72.075 45.24375) (end 73.1905 44.12825) (width 0.381) (layer "B.Cu") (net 10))
 (segment (start 89.153 56.60925) (end 88.74375 56.2) (width 0.381) (layer "B.Cu") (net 10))
 (segment (start 69.2125 57.15) (end 70.03125 57.96875) (width 0.381) (layer "B.Cu") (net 7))
 (segment (start 84.628 57.840054) (end 84.628 55.70325) (width 0.381) (layer "B.Cu") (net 7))
 (segment (start 73.7875 45.43125) (end 73.975 45.24375) (width 0.381) (layer "B.Cu") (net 7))
 (segment (start 86.6625 51.56875) (end 83.4875 51.56875) (width 0.381) (layer "B.Cu") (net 7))
 (segment (start 85.847196 59.05925) (end 84.628 57.840054) (width 0.381) (layer "B.Cu") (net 7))
 (segment (start 84.4935 55.56875) (end 83.4875 55.56875) (width 0.381) (layer "B.Cu") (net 7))
 (segment (start 67.625 55.5625) (end 69.2125 57.15) (width 0.381) (layer "B.Cu") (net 7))
 (segment (start 48.41875 57.15) (end 50.00625 55.5625) (width 0.381) (layer "B.Cu") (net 7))
 (segment (start 50.00625 55.5625) (end 67.625 55.5625) (width 0.381) (layer "B.Cu") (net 7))
 (segment (start 73.7875 49.06875) (end 73.7875 45.43125) (width 0.381) (layer "B.Cu") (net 7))
 (segment (start 87.3125 50.91875) (end 86.6625 51.56875) (width 0.381) (layer "B.Cu") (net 7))
 (segment (start 87.147 59.05925) (end 85.847196 59.05925) (width 0.381) (layer "B.Cu") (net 7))
 (segment (start 84.628 55.70325) (end 84.4935 55.56875) (width 0.381) (layer "B.Cu") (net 7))
 (segment (start 88.2625 57.94375) (end 87.147 59.05925) (width 0.381) (layer "B.Cu") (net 7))
 (segment (start 48.41875 56.9625) (end 48.41875 57.15) (width 0.381) (layer "B.Cu") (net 7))
 (segment (start 70.03125 57.96875) (end 72.0875 57.96875) (width 0.381) (layer "B.Cu") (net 7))
 (segment (start 78.5875 60.46875) (end 78.5875 63.01875) (width 0.25) (layer "B.Cu") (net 12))
 (segment (start 79.8625 64.29375) (end 84.775 64.29375) (width 0.25) (layer "B.Cu") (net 12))
 (segment (start 76.6875 67.46875) (end 79.8625 64.29375) (width 0.25) (layer "B.Cu") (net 12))
 (segment (start 78.5875 63.01875) (end 79.8625 64.29375) (width 0.25) (layer "B.Cu") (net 12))
 (segment (start 69.85 67.575673) (end 69.85 65.24375) (width 0.25) (layer "B.Cu") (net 11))
 (segment (start 72.368077 70.09375) (end 69.85 67.575673) (width 0.25) (layer "B.Cu") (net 11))
 (segment (start 78.8875 69.16875) (end 77.9625 70.09375) (width 0.25) (layer "B.Cu") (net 11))
 (segment (start 69.85 65.24375) (end 73.8875 65.24375) (width 0.25) (layer "B.Cu") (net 11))
 (segment (start 77.9625 70.09375) (end 72.368077 70.09375) (width 0.25) (layer "B.Cu") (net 11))
 (segment (start 77.7875 61.34375) (end 77.7875 60.46875) (width 0.25) (layer "B.Cu") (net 11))
 (segment (start 73.8875 65.24375) (end 77.7875 61.34375) (width 0.25) (layer "B.Cu") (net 11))
 (segment (start 51.74 44.38125) (end 48.41875 47.7025) (width 0.381) (layer "F.Cu") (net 9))
 (segment (start 48.41875 47.7025) (end 48.41875 53.975) (width 0.381) (layer "F.Cu") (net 9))
 (segment (start 68.2625 50.68125) (end 68.35 50.76875) (width 0.25) (layer "B.Cu") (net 19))
 (segment (start 68.35 50.76875) (end 72.0875 50.76875) (width 0.25) (layer "B.Cu") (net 19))
 (segment (start 53.47853 41.80625) (end 54.50625 41.80625) (width 0.2) (layer "F.Cu") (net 16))
 (segment (start 56.35625 43.65625) (end 56.35625 50.00625) (width 0.2) (layer "F.Cu") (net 16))
 (segment (start 54.50625 41.80625) (end 56.35625 43.65625) (width 0.2) (layer "F.Cu") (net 16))
 (segment (start 52.54 42.74478) (end 53.47853 41.80625) (width 0.2) (layer "F.Cu") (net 16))
 (segment (start 52.54 43.18125) (end 52.54 42.74478) (width 0.2) (layer "F.Cu") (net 16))
 (segment (start 82.3875 47.99375) (end 82.3875 52.14375) (width 0.25) (layer "B.Cu") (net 18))
 (segment (start 82.6125 52.36875) (end 83.4875 52.36875) (width 0.25) (layer "B.Cu") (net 18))
 (segment (start 61.0435 43.61275) (end 78.0065 43.61275) (width 0.25) (layer "B.Cu") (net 18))
 (segment (start 78.0065 43.61275) (end 82.3875 47.99375) (width 0.25) (layer "B.Cu") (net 18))
 (segment (start 56.35625 48.3) (end 61.0435 43.61275) (width 0.25) (layer "B.Cu") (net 18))
 (segment (start 82.3875 52.14375) (end 82.6125 52.36875) (width 0.25) (layer "B.Cu") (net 18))
 (segment (start 53.34 44.38125) (end 53.34 48.26) (width 0.2) (layer "F.Cu") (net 15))
 (segment (start 53.34 48.26) (end 51.59375 50.00625) (width 0.2) (layer "F.Cu") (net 15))
 (segment (start 88.3375 51.419423) (end 86.588173 53.16875) (width 0.25) (layer "B.Cu") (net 23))
 (segment (start 51.59375 48.3) (end 52.43125 47.4625) (width 0.25) (layer "B.Cu") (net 23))
 (segment (start 52.43125 47.4625) (end 56.557354 47.4625) (width 0.25) (layer "B.Cu") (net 23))
 (segment (start 56.557354 47.4625) (end 60.857104 43.16275) (width 0.25) (layer "B.Cu") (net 23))
 (segment (start 86.588173 53.16875) (end 83.4875 53.16875) (width 0.25) (layer "B.Cu") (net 23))
 (segment (start 88.000673 50.08125) (end 88.3375 50.418077) (width 0.25) (layer "B.Cu") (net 23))
 (segment (start 88.3375 50.418077) (end 88.3375 51.419423) (width 0.25) (layer "B.Cu") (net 23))
 (segment (start 86.624327 50.08125) (end 88.000673 50.08125) (width 0.25) (layer "B.Cu") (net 23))
 (segment (start 79.705827 43.16275) (end 86.624327 50.08125) (width 0.25) (layer "B.Cu") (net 23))
 (segment (start 60.857104 43.16275) (end 79.705827 43.16275) (width 0.25) (layer "B.Cu") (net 23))
 (segment (start 73.1875 61.54375) (end 73.1875 59.39375) (width 0.25) (layer "B.Cu") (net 8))
 (segment (start 57.86875 68.79375) (end 62.36875 64.29375) (width 0.25) (layer "B.Cu") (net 8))
 (segment (start 62.36875 64.29375) (end 70.4375 64.29375) (width 0.25) (layer "B.Cu") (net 8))
 (segment (start 80.7875 59.39375) (end 81.1875 59.79375) (width 0.25) (layer "B.Cu") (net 8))
 (segment (start 81.1875 59.79375) (end 81.1875 61.11875) (width 0.25) (layer "B.Cu") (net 8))
 (segment (start 73.1875 59.39375) (end 80.7875 59.39375) (width 0.25) (layer "B.Cu") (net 8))
 (segment (start 70.4375 64.29375) (end 73.1875 61.54375) (width 0.25) (layer "B.Cu") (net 8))
 (segment (start 81.1875 61.11875) (end 80.9875 60.91875) (width 0.25) (layer "B.Cu") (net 8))
 (segment (start 80.9875 60.91875) (end 80.9875 60.46875) (width 0.25) (layer "B.Cu") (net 8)))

